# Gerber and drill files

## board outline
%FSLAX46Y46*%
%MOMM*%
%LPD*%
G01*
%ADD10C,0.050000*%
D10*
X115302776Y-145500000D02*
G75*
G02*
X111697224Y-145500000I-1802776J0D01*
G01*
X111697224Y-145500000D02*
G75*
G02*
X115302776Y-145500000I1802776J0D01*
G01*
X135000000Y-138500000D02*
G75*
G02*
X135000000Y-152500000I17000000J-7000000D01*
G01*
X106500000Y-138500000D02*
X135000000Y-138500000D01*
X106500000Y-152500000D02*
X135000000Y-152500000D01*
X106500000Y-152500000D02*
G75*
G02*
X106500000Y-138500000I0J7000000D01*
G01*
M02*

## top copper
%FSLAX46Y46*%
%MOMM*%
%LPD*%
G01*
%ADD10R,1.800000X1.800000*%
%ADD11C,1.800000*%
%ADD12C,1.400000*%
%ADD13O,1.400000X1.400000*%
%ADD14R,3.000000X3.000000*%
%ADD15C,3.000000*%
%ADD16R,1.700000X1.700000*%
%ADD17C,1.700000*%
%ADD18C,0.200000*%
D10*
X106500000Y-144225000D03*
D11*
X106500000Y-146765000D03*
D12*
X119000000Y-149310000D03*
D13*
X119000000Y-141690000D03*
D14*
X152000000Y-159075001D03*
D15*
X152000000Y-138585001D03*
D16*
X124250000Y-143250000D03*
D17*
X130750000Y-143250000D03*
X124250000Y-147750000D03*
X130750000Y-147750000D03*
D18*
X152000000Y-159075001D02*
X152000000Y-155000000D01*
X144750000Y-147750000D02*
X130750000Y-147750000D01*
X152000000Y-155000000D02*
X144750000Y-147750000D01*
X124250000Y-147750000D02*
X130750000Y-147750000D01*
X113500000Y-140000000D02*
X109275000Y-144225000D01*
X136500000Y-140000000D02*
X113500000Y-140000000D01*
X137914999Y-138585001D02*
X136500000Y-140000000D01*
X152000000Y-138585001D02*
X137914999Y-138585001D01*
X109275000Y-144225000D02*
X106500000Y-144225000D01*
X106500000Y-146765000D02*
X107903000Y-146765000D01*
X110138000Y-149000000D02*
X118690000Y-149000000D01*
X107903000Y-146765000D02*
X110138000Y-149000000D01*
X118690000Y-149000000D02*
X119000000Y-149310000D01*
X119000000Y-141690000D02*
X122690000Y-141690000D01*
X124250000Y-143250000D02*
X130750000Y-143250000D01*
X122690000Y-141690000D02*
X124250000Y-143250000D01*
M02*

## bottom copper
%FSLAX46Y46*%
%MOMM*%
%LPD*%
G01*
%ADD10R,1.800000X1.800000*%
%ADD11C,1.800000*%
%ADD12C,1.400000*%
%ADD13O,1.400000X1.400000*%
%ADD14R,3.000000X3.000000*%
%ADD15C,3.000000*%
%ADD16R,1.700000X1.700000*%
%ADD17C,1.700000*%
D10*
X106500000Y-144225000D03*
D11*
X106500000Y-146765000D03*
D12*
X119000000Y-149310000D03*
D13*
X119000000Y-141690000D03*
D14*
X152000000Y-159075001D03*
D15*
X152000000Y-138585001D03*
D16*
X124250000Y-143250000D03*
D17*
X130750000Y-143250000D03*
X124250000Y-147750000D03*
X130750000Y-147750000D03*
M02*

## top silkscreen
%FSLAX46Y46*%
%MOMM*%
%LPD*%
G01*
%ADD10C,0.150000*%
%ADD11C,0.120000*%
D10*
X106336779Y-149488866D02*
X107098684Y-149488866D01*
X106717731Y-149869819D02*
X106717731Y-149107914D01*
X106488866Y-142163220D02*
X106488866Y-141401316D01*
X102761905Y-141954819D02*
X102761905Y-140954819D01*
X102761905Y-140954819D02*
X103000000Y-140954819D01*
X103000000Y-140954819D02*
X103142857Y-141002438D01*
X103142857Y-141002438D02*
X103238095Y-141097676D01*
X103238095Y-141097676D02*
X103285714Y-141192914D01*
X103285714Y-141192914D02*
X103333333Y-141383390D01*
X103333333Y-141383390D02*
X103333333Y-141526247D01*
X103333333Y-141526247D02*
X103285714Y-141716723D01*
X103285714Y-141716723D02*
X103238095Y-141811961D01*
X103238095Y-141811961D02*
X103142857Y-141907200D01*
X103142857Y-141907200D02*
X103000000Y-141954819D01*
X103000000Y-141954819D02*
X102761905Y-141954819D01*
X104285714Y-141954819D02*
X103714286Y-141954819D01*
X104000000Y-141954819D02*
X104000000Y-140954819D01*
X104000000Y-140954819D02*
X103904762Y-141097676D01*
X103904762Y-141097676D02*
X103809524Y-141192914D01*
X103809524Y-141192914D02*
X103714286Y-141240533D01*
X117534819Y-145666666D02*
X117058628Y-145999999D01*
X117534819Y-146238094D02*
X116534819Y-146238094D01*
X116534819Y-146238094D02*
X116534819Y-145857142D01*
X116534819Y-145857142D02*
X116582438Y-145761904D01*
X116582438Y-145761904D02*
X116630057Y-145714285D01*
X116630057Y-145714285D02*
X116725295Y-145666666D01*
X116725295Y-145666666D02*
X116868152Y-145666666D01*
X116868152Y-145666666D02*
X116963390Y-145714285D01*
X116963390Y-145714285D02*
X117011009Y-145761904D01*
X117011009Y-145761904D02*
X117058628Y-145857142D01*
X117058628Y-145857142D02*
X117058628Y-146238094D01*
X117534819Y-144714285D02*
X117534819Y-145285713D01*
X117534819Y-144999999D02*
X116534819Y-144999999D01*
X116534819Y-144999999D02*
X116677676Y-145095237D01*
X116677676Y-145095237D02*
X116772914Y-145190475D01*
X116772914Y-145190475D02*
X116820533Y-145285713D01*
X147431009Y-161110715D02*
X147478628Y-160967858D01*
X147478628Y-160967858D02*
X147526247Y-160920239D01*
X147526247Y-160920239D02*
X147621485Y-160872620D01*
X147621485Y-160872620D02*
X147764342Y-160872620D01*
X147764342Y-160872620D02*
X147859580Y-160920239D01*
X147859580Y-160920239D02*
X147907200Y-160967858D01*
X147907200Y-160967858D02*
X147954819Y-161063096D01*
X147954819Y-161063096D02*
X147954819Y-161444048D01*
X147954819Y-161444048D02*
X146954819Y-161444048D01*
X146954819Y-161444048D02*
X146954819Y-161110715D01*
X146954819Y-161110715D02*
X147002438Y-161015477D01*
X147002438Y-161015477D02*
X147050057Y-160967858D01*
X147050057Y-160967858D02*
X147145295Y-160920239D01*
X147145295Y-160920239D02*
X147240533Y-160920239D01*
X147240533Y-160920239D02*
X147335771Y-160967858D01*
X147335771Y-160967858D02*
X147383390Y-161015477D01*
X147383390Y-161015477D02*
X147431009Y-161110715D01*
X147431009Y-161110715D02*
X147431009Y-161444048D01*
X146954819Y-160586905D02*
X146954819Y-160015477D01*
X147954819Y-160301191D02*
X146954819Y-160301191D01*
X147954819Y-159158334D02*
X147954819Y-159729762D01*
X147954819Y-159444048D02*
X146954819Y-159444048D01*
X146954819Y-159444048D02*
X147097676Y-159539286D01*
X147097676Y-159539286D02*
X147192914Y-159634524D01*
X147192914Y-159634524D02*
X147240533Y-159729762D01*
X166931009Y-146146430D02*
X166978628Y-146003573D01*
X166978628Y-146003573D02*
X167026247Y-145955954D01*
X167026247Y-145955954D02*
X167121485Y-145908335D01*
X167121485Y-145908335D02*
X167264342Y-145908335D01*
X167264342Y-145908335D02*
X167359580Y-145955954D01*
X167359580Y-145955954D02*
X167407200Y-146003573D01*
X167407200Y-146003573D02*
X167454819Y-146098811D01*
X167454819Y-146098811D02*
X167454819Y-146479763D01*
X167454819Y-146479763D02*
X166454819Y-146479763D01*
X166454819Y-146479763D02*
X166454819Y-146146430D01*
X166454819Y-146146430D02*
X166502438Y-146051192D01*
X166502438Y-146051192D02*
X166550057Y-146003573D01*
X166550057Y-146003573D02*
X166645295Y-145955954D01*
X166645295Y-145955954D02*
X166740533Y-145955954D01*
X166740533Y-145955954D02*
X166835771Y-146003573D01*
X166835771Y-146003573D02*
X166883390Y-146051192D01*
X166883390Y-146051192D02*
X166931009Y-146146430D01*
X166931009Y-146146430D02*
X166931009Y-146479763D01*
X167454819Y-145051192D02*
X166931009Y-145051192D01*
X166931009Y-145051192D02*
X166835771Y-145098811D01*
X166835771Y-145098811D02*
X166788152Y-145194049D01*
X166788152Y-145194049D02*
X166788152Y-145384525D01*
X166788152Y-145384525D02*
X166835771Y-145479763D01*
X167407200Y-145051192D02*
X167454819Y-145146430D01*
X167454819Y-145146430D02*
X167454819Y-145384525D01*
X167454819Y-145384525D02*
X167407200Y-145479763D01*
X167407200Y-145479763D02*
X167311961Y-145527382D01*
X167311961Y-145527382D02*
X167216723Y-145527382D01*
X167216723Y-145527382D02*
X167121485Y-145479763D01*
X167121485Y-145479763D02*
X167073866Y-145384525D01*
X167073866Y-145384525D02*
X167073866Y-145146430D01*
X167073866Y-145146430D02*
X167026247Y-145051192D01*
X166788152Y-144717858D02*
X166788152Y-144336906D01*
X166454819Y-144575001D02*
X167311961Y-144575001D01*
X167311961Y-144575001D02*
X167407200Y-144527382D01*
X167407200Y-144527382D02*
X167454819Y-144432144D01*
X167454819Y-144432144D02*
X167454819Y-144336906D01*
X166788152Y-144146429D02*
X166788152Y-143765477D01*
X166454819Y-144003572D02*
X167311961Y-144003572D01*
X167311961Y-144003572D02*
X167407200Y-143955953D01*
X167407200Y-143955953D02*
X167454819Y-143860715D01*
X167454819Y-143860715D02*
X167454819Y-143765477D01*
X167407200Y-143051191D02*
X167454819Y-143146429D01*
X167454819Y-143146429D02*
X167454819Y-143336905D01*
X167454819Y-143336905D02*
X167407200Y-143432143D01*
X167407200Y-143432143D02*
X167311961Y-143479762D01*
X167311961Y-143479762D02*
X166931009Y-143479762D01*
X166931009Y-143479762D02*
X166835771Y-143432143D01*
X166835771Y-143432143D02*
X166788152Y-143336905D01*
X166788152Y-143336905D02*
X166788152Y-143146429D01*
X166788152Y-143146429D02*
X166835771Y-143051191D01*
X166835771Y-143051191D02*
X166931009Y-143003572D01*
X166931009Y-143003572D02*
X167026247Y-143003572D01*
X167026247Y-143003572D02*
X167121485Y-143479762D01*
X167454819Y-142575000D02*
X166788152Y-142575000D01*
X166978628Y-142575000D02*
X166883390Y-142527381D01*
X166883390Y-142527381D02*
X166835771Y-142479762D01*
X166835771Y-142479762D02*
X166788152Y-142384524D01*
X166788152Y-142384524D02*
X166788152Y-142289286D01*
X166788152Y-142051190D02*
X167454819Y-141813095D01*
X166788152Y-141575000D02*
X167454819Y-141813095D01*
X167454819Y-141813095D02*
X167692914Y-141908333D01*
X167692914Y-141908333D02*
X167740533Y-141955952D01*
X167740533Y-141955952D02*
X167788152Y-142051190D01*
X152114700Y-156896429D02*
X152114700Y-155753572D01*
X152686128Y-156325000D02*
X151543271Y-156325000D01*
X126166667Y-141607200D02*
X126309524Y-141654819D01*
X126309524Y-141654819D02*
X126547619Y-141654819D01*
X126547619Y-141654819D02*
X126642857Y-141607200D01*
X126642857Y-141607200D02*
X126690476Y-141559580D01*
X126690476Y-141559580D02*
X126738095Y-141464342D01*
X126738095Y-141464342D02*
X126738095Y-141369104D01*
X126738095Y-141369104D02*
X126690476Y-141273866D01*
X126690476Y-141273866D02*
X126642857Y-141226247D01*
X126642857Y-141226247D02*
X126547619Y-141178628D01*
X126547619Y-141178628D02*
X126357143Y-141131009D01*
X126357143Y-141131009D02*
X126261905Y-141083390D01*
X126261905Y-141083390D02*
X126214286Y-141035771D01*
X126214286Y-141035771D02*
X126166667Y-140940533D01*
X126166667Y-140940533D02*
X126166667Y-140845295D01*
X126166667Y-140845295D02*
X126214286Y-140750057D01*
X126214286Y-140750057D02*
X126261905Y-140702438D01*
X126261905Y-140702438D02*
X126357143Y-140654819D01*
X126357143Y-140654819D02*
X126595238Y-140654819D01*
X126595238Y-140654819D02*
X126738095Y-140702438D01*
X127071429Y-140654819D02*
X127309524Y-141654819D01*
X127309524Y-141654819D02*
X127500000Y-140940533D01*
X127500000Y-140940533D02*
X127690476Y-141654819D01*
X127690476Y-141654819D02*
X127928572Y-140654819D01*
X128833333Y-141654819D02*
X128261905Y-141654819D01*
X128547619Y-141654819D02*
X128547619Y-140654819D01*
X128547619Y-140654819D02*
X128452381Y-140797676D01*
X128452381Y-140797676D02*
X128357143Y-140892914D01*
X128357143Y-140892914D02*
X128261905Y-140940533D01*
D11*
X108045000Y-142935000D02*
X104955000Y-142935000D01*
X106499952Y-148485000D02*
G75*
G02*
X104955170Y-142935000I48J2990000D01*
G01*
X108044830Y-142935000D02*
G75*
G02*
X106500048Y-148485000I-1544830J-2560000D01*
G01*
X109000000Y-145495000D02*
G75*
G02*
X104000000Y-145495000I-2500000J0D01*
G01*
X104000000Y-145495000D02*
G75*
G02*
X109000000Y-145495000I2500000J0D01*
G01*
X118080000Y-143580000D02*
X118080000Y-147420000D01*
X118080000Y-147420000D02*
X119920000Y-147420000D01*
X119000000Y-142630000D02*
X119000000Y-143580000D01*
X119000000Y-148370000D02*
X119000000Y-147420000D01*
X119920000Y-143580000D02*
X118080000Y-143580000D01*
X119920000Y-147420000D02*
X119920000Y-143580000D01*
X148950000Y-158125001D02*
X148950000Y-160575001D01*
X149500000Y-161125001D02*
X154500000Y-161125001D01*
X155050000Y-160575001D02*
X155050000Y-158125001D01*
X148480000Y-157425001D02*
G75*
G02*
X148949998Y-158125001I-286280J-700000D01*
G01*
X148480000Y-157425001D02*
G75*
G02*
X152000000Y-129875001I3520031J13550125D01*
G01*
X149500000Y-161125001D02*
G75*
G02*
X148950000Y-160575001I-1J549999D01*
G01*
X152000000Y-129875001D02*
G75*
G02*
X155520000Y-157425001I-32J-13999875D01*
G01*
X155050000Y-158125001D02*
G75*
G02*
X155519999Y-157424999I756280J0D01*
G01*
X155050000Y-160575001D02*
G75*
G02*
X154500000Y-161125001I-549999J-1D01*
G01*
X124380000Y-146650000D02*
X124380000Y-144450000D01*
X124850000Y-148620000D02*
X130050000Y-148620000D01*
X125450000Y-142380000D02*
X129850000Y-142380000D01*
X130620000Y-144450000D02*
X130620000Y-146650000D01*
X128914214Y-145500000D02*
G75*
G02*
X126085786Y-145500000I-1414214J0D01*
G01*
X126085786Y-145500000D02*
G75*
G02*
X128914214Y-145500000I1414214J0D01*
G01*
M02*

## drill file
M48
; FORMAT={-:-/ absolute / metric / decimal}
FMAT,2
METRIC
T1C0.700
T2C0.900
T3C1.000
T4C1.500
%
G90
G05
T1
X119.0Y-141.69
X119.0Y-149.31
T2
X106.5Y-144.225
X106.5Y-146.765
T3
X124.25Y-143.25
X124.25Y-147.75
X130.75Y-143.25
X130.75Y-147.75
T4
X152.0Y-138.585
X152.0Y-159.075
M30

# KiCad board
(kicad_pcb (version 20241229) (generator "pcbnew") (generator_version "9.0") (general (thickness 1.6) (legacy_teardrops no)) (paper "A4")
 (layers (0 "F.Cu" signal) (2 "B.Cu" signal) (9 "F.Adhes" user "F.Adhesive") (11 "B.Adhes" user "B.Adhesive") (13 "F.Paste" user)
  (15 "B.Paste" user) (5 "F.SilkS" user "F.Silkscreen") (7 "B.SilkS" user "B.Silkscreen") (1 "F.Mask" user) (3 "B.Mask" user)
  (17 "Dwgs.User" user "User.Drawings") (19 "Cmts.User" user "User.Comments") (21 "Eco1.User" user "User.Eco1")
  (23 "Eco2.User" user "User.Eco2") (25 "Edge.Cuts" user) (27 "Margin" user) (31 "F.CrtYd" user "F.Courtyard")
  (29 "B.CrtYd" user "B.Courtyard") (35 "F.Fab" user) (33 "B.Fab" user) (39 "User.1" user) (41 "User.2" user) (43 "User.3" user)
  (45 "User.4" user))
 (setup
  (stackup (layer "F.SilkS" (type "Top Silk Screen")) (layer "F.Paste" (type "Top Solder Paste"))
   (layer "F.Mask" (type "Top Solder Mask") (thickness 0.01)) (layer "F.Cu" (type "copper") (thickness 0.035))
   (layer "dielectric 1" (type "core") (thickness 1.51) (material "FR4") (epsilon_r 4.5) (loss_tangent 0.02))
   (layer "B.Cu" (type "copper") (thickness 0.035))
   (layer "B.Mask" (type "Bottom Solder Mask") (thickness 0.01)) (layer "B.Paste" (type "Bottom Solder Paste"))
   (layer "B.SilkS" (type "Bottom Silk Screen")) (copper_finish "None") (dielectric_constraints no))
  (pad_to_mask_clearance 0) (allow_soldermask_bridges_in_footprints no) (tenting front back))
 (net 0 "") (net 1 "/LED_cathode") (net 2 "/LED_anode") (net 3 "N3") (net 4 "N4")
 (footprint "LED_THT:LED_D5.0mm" (layer "F.Cu") (at 106.5 144.225 -90)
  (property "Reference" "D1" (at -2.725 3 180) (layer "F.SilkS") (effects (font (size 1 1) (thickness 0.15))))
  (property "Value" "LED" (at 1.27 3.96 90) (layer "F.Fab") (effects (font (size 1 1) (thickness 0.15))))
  (fp_line (start -1.29 -1.545) (end -1.29 1.545) (stroke (width 0.12) (type solid)) (layer "F.SilkS"))
  (fp_arc (start 4.26 0.000048) (mid 2.071756 2.880501) (end -1.29 1.54483) (stroke (width 0.12) (type solid)) (layer "F.SilkS"))
  (fp_arc (start -1.29 -1.54483) (mid 2.071756 -2.880501) (end 4.26 -0.000048) (stroke (width 0.12) (type solid)) (layer "F.SilkS"))
  (fp_circle (center 1.27 0) (end 3.77 0) (stroke (width 0.12) (type solid)) (fill no) (layer "F.SilkS"))
  (pad "1" thru_hole rect (at 0 0 270) (size 1.8 1.8) (drill 0.9) (layers "*.Cu" "*.Mask") (remove_unused_layers no) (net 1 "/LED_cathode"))
  (pad "2" thru_hole circle (at 2.54 0 270) (size 1.8 1.8) (drill 0.9) (layers "*.Cu" "*.Mask") (remove_unused_layers no)
   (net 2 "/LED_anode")))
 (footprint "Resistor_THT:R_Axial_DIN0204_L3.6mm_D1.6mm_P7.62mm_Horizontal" (layer "F.Cu") (at 119 149.31 90)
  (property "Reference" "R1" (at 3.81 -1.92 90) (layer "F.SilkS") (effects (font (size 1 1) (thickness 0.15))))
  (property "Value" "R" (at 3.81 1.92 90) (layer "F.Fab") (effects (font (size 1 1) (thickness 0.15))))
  (fp_line (start 5.73 -0.92) (end 1.89 -0.92) (stroke (width 0.12) (type solid)) (layer "F.SilkS"))
  (fp_line (start 1.89 -0.92) (end 1.89 0.92) (stroke (width 0.12) (type solid)) (layer "F.SilkS"))
  (fp_line (start 6.68 0) (end 5.73 0) (stroke (width 0.12) (type solid)) (layer "F.SilkS"))
  (fp_line (start 0.94 0) (end 1.89 0) (stroke (width 0.12) (type solid)) (layer "F.SilkS"))
  (fp_line (start 5.73 0.92) (end 5.73 -0.92) (stroke (width 0.12) (type solid)) (layer "F.SilkS"))
  (fp_line (start 1.89 0.92) (end 5.73 0.92) (stroke (width 0.12) (type solid)) (layer "F.SilkS"))
  (pad "1" thru_hole circle (at 0 0 90) (size 1.4 1.4) (drill 0.7) (layers "*.Cu" "*.Mask") (remove_unused_layers no) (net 2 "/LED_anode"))
  (pad "2" thru_hole oval (at 7.62 0 90) (size 1.4 1.4) (drill 0.7) (layers "*.Cu" "*.Mask") (remove_unused_layers no) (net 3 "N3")))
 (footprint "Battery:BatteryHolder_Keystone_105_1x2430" (layer "F.Cu") (at 152 159.075001 90)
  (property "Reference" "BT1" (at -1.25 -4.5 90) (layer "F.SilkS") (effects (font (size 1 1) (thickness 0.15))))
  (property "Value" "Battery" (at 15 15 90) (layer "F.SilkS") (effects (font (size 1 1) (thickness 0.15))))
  (fp_line (start 0.95 -3.05) (end -1.5 -3.05) (stroke (width 0.12) (type solid)) (layer "F.SilkS"))
  (fp_line (start -2.05 -2.5) (end -2.05 2.5) (stroke (width 0.12) (type solid)) (layer "F.SilkS"))
  (fp_line (start -1.5 3.05) (end 0.95 3.05) (stroke (width 0.12) (type solid)) (layer "F.SilkS"))
  (fp_arc (start 1.65 -3.52) (mid 1.371575 -3.1784) (end 0.95 -3.05) (stroke (width 0.12) (type solid)) (layer "F.SilkS"))
  (fp_arc (start 1.65 -3.52) (mid 16.974433 -13.886953) (end 29.2 0) (stroke (width 0.12) (type solid)) (layer "F.SilkS"))
  (fp_arc (start -2.05 -2.5) (mid -1.888909 -2.888909) (end -1.5 -3.05) (stroke (width 0.12) (type solid)) (layer "F.SilkS"))
  (fp_arc (start 29.2 0) (mid 16.974433 13.886952) (end 1.65 3.52) (stroke (width 0.12) (type solid)) (layer "F.SilkS"))
  (fp_arc (start 0.95 3.05) (mid 1.371574 3.1784) (end 1.65 3.52) (stroke (width 0.12) (type solid)) (layer "F.SilkS"))
  (fp_arc (start -1.5 3.05) (mid -1.888909 2.888909) (end -2.05 2.5) (stroke (width 0.12) (type solid)) (layer "F.SilkS"))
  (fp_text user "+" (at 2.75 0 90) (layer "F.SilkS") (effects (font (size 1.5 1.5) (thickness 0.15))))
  (pad "1" thru_hole rect (at 0 0 90) (size 3 3) (drill 1.5) (layers "*.Cu" "*.Mask") (remove_unused_layers no) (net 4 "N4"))
  (pad "2" thru_hole circle (at 20.49 0 90) (size 3 3) (drill 1.5) (layers "*.Cu" "*.Mask") (remove_unused_layers no) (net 1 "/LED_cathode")))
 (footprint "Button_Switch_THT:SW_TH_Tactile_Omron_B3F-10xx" (layer "F.Cu") (at 124.25 143.25)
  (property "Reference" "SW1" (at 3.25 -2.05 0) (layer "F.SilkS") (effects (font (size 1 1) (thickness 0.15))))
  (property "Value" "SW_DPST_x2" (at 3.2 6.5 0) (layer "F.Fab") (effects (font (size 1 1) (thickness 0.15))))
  (fp_line (start 0.13 3.4) (end 0.13 1.2) (stroke (width 0.12) (type solid)) (layer "F.SilkS"))
  (fp_line (start 0.6 5.37) (end 5.8 5.37) (stroke (width 0.12) (type solid)) (layer "F.SilkS"))
  (fp_line (start 1.2 -0.87) (end 5.6 -0.87) (stroke (width 0.12) (type solid)) (layer "F.SilkS"))
  (fp_line (start 6.37 1.2) (end 6.37 3.4) (stroke (width 0.12) (type solid)) (layer "F.SilkS"))
  (fp_circle (center 3.25 2.25) (end 4.25 3.25) (stroke (width 0.12) (type solid)) (fill no) (layer "F.SilkS"))
  (pad "1" thru_hole rect (at 0 0) (size 1.7 1.7) (drill 1) (layers "*.Cu" "*.Mask") (remove_unused_layers no) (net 3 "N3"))
  (pad "1" thru_hole circle (at 6.5 0) (size 1.7 1.7) (drill 1) (layers "*.Cu" "*.Mask") (remove_unused_layers no) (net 3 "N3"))
  (pad "2" thru_hole circle (at 0 4.5) (size 1.7 1.7) (drill 1) (layers "*.Cu" "*.Mask") (remove_unused_layers no) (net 4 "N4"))
  (pad "2" thru_hole circle (at 6.5 4.5) (size 1.7 1.7) (drill 1) (layers "*.Cu" "*.Mask") (remove_unused_layers no) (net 4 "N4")))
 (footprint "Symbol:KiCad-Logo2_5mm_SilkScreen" (layer "B.Cu") (at 152 144 180)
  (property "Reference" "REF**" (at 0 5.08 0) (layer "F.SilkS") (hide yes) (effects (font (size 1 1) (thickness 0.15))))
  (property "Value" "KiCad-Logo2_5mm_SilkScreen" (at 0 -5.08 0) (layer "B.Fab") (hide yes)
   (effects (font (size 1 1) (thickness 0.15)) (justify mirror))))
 (gr_circle (center 113.5 145.5) (end 114.5 147) (stroke (width 0.05) (type default)) (fill no) (layer "Edge.Cuts"))
 (gr_arc (start 135 138.5) (mid 170.384776 145.5) (end 135 152.5) (stroke (width 0.05) (type default)) (layer "Edge.Cuts"))
 (gr_line (start 106.5 138.5) (end 135 138.5) (stroke (width 0.05) (type default)) (layer "Edge.Cuts"))
 (gr_line (start 106.5 152.5) (end 135 152.5) (stroke (width 0.05) (type default)) (layer "Edge.Cuts"))
 (gr_arc (start 106.5 152.5) (mid 99.5 145.5) (end 106.5 138.5) (stroke (width 0.05) (type default)) (layer "Edge.Cuts"))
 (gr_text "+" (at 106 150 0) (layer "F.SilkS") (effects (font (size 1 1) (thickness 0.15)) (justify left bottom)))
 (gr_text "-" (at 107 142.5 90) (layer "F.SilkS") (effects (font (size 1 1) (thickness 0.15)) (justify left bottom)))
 (segment (start 152 159.075001) (end 152 155) (width 0.2) (layer "F.Cu") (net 4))
 (segment (start 144.75 147.75) (end 130.75 147.75) (width 0.2) (layer "F.Cu") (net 4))
 (segment (start 152 155) (end 144.75 147.75) (width 0.2) (layer "F.Cu") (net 4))
 (segment (start 124.25 147.75) (end 130.75 147.75) (width 0.2) (layer "F.Cu") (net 4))
 (segment (start 113.5 140) (end 109.275 144.225) (width 0.2) (layer "F.Cu") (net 1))
 (segment (start 136.5 140) (end 113.5 140) (width 0.2) (layer "F.Cu") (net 1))
 (segment (start 137.914999 138.585001) (end 136.5 140) (width 0.2) (layer "F.Cu") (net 1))
 (segment (start 152 138.585001) (end 137.914999 138.585001) (width 0.2) (layer "F.Cu") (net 1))
 (segment (start 109.275 144.225) (end 106.5 144.225) (width 0.2) (layer "F.Cu") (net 1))
 (segment (start 106.5 146.765) (end 107.903 146.765) (width 0.2) (layer "F.Cu") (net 2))
 (segment (start 110.138 149) (end 118.69 149) (width 0.2) (layer "F.Cu") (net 2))
 (segment (start 107.903 146.765) (end 110.138 149) (width 0.2) (layer "F.Cu") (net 2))
 (segment (start 118.69 149) (end 119 149.31) (width 0.2) (layer "F.Cu") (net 2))
 (segment (start 119 141.69) (end 122.69 141.69) (width 0.2) (layer "F.Cu") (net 3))
 (segment (start 124.25 143.25) (end 130.75 143.25) (width 0.2) (layer "F.Cu") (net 3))
 (segment (start 122.69 141.69) (end 124.25 143.25) (width 0.2) (layer "F.Cu") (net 3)))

